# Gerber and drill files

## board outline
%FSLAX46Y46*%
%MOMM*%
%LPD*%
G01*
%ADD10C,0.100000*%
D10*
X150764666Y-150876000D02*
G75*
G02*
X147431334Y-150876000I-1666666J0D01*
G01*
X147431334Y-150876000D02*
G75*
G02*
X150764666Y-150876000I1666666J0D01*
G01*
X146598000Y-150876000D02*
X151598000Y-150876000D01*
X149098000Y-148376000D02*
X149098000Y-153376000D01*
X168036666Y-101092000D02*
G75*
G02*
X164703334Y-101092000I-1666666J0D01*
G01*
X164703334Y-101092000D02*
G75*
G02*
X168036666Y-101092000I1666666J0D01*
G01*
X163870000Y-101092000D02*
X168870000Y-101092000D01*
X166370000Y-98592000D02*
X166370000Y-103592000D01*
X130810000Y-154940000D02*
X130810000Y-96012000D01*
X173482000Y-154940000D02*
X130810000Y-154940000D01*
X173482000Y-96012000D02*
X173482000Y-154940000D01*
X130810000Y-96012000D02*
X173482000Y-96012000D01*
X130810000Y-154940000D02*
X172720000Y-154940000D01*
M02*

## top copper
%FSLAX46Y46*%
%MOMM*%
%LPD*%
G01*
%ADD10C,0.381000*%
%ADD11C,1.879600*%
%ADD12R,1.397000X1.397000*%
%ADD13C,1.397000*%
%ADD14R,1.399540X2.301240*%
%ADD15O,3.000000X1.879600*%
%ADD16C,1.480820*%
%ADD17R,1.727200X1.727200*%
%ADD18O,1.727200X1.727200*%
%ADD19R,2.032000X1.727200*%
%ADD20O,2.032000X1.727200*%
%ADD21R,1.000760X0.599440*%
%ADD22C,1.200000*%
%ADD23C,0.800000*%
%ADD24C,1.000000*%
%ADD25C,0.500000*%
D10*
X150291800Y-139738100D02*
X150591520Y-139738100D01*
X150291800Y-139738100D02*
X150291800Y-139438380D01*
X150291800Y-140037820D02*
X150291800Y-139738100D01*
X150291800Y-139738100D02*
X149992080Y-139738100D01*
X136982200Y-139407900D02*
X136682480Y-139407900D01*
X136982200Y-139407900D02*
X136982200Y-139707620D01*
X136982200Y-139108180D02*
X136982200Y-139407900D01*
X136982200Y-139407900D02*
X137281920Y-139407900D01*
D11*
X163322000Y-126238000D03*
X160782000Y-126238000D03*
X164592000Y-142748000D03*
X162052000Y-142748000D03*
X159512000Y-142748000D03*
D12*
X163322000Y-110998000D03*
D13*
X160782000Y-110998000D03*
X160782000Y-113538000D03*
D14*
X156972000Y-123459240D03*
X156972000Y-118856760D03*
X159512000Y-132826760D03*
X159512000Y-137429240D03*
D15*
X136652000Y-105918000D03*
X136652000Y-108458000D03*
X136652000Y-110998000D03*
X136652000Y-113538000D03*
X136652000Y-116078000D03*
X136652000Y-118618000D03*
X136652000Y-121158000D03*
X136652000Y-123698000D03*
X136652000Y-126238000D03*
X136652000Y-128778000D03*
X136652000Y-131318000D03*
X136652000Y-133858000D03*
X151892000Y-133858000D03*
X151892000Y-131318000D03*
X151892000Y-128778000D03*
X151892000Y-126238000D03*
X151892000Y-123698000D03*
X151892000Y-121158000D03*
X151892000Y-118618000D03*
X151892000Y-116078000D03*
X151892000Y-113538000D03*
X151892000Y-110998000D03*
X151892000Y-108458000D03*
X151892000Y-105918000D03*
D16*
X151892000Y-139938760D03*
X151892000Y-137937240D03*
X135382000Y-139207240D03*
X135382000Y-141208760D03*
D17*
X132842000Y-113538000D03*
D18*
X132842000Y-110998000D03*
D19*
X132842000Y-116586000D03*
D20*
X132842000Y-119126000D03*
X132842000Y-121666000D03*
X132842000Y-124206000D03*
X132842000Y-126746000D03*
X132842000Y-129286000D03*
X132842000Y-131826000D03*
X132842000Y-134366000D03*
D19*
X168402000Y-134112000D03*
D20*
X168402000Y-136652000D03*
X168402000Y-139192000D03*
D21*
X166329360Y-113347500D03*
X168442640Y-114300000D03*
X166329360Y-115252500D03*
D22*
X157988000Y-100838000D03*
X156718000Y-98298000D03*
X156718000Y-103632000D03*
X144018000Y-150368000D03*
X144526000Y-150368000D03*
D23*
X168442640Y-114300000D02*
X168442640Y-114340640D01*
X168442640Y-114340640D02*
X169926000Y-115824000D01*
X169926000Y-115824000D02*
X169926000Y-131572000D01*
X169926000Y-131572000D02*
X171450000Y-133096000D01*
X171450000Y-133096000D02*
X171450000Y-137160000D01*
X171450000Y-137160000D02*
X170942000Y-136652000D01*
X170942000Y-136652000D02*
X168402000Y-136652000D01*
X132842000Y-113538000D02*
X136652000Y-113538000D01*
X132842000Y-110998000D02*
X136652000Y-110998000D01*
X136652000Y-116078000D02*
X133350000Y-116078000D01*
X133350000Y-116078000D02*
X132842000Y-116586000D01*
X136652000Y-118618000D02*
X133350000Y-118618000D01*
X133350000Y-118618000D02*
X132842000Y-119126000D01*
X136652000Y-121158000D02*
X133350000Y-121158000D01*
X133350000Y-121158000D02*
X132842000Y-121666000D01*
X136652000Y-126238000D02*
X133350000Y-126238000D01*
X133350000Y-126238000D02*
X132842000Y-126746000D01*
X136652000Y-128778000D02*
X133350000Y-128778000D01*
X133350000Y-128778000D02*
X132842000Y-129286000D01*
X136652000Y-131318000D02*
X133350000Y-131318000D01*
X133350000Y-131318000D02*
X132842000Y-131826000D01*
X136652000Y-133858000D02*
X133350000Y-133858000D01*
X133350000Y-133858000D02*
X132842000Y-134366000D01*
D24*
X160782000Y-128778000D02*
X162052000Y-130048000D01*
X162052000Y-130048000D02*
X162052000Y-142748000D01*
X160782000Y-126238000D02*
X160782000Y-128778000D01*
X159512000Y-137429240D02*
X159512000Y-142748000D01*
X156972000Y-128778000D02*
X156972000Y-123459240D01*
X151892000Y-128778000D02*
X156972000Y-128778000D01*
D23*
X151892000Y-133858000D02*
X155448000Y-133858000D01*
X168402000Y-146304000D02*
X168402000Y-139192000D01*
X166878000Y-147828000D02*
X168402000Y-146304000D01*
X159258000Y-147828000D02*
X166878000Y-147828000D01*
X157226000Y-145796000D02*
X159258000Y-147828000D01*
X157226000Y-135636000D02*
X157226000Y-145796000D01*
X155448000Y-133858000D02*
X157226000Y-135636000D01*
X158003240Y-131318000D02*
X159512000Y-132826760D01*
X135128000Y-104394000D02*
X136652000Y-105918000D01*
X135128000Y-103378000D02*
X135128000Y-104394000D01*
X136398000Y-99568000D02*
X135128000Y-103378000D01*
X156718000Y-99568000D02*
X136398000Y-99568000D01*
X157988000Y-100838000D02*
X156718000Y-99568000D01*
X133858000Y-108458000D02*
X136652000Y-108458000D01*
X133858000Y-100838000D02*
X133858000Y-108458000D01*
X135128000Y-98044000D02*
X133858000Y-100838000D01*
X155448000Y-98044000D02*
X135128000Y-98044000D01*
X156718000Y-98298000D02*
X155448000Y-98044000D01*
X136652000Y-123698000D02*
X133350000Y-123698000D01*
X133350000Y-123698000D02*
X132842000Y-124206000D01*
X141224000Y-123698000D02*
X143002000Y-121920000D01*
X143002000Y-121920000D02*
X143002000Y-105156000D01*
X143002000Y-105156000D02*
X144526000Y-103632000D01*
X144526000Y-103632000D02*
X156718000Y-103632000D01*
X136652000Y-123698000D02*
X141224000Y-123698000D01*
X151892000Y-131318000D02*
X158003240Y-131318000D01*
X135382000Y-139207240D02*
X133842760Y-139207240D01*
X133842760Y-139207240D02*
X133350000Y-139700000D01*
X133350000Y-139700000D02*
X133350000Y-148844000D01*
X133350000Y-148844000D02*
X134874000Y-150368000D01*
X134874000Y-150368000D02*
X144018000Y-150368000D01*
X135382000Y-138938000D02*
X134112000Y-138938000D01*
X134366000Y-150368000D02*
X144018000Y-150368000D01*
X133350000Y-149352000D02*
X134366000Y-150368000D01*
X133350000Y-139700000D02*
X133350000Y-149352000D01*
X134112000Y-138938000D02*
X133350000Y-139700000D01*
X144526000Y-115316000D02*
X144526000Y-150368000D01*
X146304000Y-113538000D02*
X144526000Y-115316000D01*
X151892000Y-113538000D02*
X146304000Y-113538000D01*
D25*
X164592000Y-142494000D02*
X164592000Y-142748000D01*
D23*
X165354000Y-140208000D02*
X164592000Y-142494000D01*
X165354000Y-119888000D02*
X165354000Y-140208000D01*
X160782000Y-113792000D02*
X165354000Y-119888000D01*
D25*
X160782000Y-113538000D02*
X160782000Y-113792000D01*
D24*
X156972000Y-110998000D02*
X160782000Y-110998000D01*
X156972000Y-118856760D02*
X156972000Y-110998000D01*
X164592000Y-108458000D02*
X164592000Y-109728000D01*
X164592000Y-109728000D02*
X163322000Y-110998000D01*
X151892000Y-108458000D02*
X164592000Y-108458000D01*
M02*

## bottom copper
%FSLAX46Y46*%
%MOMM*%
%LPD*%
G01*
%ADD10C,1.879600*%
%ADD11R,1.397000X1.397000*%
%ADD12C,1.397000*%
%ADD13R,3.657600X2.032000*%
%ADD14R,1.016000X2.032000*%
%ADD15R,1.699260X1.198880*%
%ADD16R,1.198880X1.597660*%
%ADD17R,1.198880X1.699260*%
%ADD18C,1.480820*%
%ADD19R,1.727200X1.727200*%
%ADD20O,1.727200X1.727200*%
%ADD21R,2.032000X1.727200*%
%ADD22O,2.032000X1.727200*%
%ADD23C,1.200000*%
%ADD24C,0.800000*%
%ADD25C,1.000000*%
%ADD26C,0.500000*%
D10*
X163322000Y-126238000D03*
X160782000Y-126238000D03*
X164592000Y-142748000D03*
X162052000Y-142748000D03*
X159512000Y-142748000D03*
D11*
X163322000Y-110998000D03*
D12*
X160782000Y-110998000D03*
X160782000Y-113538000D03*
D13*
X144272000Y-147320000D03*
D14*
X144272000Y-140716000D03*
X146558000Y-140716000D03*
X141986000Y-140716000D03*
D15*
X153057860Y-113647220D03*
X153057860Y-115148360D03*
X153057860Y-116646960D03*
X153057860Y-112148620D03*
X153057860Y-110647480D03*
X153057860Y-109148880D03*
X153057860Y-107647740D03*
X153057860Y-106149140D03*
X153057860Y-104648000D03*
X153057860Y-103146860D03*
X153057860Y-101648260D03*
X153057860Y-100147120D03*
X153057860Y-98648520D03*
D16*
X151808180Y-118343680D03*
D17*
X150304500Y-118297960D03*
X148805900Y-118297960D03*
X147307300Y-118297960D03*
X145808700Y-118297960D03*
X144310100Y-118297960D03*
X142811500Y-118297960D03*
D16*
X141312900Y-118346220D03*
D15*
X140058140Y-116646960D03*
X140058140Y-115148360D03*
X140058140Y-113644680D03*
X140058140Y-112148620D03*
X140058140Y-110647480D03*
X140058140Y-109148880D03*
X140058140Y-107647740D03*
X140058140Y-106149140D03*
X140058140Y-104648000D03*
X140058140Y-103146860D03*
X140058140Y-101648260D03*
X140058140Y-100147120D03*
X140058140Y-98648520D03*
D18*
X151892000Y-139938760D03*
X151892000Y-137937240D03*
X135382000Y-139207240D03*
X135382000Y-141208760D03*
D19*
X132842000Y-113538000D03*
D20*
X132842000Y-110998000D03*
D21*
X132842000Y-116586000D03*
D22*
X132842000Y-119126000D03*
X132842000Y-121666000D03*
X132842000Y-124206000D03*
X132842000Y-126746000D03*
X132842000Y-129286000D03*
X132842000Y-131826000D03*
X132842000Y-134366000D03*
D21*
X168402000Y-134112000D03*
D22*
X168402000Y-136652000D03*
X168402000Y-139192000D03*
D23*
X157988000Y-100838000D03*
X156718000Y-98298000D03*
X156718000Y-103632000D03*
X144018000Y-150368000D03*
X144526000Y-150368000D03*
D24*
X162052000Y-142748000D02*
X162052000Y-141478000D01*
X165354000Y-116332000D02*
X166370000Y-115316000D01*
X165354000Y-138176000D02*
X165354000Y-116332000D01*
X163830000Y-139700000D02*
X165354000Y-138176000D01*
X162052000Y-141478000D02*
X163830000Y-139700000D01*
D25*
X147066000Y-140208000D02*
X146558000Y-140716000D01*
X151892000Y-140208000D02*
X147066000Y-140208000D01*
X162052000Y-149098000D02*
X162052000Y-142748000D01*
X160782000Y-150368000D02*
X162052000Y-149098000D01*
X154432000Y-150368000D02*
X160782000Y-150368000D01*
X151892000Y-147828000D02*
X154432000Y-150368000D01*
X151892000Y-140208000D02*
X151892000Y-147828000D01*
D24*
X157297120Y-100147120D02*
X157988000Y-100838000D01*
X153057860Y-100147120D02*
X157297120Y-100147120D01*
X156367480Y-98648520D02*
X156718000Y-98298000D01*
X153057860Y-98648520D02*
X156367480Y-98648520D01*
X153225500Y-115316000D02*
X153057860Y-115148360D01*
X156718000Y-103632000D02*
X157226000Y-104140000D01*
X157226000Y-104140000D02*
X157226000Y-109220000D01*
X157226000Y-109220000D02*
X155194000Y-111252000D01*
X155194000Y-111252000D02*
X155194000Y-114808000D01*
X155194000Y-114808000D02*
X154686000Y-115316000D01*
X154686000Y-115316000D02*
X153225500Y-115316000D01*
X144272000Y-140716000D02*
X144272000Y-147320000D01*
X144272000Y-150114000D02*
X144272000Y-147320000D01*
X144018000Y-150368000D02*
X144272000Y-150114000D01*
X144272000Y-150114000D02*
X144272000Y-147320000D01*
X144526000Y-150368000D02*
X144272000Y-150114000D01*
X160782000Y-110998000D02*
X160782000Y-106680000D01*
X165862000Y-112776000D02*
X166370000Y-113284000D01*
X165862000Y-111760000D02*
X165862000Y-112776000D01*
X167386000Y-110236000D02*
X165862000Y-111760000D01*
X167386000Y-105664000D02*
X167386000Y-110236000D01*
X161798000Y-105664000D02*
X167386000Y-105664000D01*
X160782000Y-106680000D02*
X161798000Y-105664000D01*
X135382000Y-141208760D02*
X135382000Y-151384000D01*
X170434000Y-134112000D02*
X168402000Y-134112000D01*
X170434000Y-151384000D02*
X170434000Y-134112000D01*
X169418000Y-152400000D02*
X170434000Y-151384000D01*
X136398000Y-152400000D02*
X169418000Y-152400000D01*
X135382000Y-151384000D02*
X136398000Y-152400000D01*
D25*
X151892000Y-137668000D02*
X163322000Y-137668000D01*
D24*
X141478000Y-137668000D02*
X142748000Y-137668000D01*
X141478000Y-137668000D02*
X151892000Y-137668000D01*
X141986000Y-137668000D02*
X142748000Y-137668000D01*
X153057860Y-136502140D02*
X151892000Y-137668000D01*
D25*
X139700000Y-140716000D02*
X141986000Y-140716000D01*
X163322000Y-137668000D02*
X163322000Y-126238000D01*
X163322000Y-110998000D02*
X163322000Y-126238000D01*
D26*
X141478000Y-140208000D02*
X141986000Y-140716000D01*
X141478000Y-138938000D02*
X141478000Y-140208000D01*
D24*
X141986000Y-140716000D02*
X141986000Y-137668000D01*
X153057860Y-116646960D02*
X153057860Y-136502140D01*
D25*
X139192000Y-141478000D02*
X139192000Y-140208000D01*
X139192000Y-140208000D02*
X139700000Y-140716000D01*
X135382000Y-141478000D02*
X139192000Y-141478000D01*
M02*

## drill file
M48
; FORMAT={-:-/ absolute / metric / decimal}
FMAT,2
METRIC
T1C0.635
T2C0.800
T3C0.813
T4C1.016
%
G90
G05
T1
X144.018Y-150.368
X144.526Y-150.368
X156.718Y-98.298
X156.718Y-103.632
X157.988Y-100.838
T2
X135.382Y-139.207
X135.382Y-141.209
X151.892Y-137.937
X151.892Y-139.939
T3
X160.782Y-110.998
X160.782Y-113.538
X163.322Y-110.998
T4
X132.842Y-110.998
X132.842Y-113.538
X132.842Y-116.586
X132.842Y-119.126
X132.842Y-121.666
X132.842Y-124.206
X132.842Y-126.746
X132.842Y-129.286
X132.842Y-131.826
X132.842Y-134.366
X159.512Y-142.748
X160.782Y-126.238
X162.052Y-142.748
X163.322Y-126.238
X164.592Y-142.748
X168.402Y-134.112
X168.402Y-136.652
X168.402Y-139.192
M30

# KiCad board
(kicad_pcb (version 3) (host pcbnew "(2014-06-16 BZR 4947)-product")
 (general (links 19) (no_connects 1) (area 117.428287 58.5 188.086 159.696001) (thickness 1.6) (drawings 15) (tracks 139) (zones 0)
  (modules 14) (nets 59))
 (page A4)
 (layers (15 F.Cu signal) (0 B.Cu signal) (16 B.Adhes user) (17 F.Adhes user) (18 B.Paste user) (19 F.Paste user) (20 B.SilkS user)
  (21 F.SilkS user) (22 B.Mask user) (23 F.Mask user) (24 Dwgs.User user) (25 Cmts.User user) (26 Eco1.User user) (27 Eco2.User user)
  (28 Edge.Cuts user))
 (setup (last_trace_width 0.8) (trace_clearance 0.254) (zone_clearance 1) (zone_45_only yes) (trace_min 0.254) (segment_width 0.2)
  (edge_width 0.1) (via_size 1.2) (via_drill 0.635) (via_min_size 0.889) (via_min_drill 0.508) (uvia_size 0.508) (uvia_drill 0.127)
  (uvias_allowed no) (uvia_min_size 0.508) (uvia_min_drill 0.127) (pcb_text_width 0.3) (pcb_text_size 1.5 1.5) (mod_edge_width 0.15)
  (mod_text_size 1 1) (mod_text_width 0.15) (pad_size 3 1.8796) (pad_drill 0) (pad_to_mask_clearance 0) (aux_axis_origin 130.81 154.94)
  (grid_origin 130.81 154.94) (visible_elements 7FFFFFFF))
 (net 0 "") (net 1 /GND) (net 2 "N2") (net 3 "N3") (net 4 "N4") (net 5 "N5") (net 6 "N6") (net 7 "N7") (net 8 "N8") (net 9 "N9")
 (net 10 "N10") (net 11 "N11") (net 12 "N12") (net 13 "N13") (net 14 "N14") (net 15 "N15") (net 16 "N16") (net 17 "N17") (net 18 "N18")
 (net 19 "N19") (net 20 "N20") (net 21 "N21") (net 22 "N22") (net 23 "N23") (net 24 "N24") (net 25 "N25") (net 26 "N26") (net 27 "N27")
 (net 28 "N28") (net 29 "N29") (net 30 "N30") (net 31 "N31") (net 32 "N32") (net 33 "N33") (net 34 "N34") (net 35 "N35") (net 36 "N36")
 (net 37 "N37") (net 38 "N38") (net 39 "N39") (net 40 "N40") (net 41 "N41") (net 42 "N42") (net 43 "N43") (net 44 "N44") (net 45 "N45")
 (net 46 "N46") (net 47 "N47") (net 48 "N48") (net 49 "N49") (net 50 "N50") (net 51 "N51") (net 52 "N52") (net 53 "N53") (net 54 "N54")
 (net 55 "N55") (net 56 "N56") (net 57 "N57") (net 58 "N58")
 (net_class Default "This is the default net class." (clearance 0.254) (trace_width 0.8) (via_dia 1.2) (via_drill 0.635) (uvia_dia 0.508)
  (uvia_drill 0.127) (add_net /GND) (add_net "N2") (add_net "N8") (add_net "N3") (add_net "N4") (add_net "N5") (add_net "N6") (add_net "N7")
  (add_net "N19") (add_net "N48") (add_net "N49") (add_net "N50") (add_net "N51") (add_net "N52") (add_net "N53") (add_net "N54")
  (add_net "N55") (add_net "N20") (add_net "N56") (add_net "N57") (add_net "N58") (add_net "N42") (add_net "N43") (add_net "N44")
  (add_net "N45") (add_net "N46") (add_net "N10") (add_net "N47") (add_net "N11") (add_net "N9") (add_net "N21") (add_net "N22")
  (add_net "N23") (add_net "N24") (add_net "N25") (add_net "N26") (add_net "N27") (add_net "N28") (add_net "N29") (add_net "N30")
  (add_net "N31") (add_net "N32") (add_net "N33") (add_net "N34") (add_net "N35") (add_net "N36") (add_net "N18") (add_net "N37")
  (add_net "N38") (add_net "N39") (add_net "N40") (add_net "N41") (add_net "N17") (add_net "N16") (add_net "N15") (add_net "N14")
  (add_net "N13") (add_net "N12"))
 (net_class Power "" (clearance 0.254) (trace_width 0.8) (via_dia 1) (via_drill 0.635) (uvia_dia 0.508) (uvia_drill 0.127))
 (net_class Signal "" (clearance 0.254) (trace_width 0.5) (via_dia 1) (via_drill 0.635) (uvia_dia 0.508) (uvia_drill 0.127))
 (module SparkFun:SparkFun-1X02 (layer F.Cu) (at 163.322 126.238 180)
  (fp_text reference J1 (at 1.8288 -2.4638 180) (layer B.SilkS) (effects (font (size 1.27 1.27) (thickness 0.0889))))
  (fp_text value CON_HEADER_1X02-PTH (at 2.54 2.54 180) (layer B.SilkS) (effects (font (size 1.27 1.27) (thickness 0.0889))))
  (pad 1 thru_hole circle (at 0 0 180) (size 1.8796 1.8796) (drill 1.016) (layers *.Cu F.Paste F.SilkS F.Mask) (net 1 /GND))
  (pad 2 thru_hole circle (at 2.54 0 180) (size 1.8796 1.8796) (drill 1.016) (layers *.Cu F.Paste F.SilkS F.Mask) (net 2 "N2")))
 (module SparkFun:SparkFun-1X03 (layer F.Cu) (at 164.592 142.748 180)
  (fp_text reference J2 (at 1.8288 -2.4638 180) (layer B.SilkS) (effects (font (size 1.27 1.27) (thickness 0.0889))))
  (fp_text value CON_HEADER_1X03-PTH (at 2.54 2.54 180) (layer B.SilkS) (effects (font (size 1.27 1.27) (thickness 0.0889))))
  (pad 1 thru_hole circle (at 0 0 180) (size 1.8796 1.8796) (drill 1.016) (layers *.Cu F.Paste F.SilkS F.Mask) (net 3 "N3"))
  (pad 2 thru_hole circle (at 2.54 0 180) (size 1.8796 1.8796) (drill 1.016) (layers *.Cu F.Paste F.SilkS F.Mask) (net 2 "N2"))
  (pad 3 thru_hole circle (at 5.08 0 180) (size 1.8796 1.8796) (drill 1.016) (layers *.Cu F.Paste F.SilkS F.Mask) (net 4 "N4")))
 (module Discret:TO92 (layer F.Cu) (at 162.052 112.268)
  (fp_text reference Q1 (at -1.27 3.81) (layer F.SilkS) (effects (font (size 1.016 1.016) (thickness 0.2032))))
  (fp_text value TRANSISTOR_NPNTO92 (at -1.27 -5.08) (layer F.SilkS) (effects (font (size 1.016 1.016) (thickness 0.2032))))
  (pad 1 thru_hole rect (at 1.27 -1.27) (size 1.397 1.397) (drill 0.8128) (layers *.Cu *.Mask F.SilkS) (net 1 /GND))
  (pad 2 thru_hole circle (at -1.27 -1.27) (size 1.397 1.397) (drill 0.8128) (layers *.Cu *.Mask F.SilkS) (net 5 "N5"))
  (pad 3 thru_hole circle (at -1.27 1.27) (size 1.397 1.397) (drill 0.8128) (layers *.Cu *.Mask F.SilkS) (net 3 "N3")))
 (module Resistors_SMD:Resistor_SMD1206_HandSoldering (layer F.Cu) (at 156.972 121.158 90)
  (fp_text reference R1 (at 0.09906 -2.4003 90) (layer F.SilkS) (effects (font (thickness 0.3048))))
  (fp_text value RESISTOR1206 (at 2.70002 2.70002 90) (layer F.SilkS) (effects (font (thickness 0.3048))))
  (pad 1 smd rect (at -2.30124 0 90) (size 2.30124 1.39954) (layers F.Cu F.Paste F.Mask) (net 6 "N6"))
  (pad 2 smd rect (at 2.30124 0 90) (size 2.30124 1.39954) (layers F.Cu F.Paste F.Mask) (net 5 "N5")))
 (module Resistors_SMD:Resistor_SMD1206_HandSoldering (layer F.Cu) (at 159.512 135.128 270)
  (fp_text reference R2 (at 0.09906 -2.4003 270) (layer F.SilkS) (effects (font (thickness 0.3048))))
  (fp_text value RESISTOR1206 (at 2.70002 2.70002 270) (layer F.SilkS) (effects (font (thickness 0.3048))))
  (pad 1 smd rect (at -2.30124 0 270) (size 2.30124 1.39954) (layers F.Cu F.Paste F.Mask) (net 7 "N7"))
  (pad 2 smd rect (at 2.30124 0 270) (size 2.30124 1.39954) (layers F.Cu F.Paste F.Mask) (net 4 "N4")))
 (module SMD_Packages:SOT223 (layer B.Cu) (at 144.272 144.018)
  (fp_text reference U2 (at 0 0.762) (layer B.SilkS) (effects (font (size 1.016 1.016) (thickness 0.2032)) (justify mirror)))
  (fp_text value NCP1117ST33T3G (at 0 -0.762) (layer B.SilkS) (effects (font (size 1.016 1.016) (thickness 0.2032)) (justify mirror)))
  (pad 4 smd rect (at 0 3.302) (size 3.6576 2.032) (layers B.Cu B.Paste B.Mask))
  (pad 2 smd rect (at 0 -3.302) (size 1.016 2.032) (layers B.Cu B.Paste B.Mask) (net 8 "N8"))
  (pad 3 smd rect (at 2.286 -3.302) (size 1.016 2.032) (layers B.Cu B.Paste B.Mask) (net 2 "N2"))
  (pad 1 smd rect (at -2.286 -3.302) (size 1.016 2.032) (layers B.Cu B.Paste B.Mask) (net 1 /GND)))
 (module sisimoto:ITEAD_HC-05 (layer B.Cu) (at 146.558 104.648 180)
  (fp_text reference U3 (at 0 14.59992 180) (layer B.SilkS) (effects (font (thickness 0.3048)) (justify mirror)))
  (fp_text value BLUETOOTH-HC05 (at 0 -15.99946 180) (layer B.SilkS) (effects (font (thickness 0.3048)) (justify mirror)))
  (pad 11 smd rect (at -6.49986 -8.99922 180) (size 1.69926 1.19888) (layers B.Cu B.Paste B.Mask) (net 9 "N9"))
  (pad 12 smd rect (at -6.49986 -10.50036 180) (size 1.69926 1.19888) (layers B.Cu B.Paste B.Mask) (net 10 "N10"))
  (pad 13 smd rect (at -6.49986 -11.99896 180) (size 1.69926 1.19888) (layers B.Cu B.Paste B.Mask) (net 1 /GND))
  (pad 10 smd rect (at -6.49986 -7.50062 180) (size 1.69926 1.19888) (layers B.Cu B.Paste B.Mask) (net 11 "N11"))
  (pad 9 smd rect (at -6.49986 -5.99948 180) (size 1.69926 1.19888) (layers B.Cu B.Paste B.Mask) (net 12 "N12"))
  (pad 8 smd rect (at -6.49986 -4.50088 180) (size 1.69926 1.19888) (layers B.Cu B.Paste B.Mask) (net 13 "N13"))
  (pad 7 smd rect (at -6.49986 -2.99974 180) (size 1.69926 1.19888) (layers B.Cu B.Paste B.Mask) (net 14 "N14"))
  (pad 6 smd rect (at -6.49986 -1.50114 180) (size 1.69926 1.19888) (layers B.Cu B.Paste B.Mask) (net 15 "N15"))
  (pad 5 smd rect (at -6.49986 0 180) (size 1.69926 1.19888) (layers B.Cu B.Paste B.Mask) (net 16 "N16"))
  (pad 4 smd rect (at -6.49986 1.50114 180) (size 1.69926 1.19888) (layers B.Cu B.Paste B.Mask) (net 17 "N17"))
  (pad 3 smd rect (at -6.49986 2.99974 180) (size 1.69926 1.19888) (layers B.Cu B.Paste B.Mask) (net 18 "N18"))
  (pad 2 smd rect (at -6.49986 4.50088 180) (size 1.69926 1.19888) (layers B.Cu B.Paste B.Mask) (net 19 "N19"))
  (pad 1 smd rect (at -6.49986 5.99948 180) (size 1.69926 1.19888) (layers B.Cu B.Paste B.Mask) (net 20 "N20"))
  (pad 14 smd rect (at -5.25018 -13.69568 180) (size 1.19888 1.59766) (layers B.Cu B.Paste B.Mask) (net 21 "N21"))
  (pad 15 smd rect (at -3.7465 -13.64996 180) (size 1.19888 1.69926) (layers B.Cu B.Paste B.Mask) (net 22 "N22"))
  (pad 16 smd rect (at -2.2479 -13.64996 180) (size 1.19888 1.69926) (layers B.Cu B.Paste B.Mask) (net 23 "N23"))
  (pad 17 smd rect (at -0.7493 -13.64996 180) (size 1.19888 1.69926) (layers B.Cu B.Paste B.Mask) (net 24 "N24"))
  (pad 18 smd rect (at 0.7493 -13.64996 180) (size 1.19888 1.69926) (layers B.Cu B.Paste B.Mask) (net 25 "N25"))
  (pad 19 smd rect (at 2.2479 -13.64996 180) (size 1.19888 1.69926) (layers B.Cu B.Paste B.Mask) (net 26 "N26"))
  (pad 20 smd rect (at 3.7465 -13.64996 180) (size 1.19888 1.69926) (layers B.Cu B.Paste B.Mask) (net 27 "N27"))
  (pad 21 smd rect (at 5.2451 -13.69822 180) (size 1.19888 1.59766) (layers B.Cu B.Paste B.Mask) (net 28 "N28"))
  (pad 22 smd rect (at 6.49986 -11.99896 180) (size 1.69926 1.19888) (layers B.Cu B.Paste B.Mask) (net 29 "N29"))
  (pad 23 smd rect (at 6.49986 -10.50036 180) (size 1.69926 1.19888) (layers B.Cu B.Paste B.Mask) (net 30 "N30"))
  (pad 24 smd rect (at 6.49986 -8.99668 180) (size 1.69926 1.19888) (layers B.Cu B.Paste B.Mask) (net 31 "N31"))
  (pad 25 smd rect (at 6.49986 -7.50062 180) (size 1.69926 1.19888) (layers B.Cu B.Paste B.Mask) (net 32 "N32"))
  (pad 26 smd rect (at 6.49986 -5.99948 180) (size 1.69926 1.19888) (layers B.Cu B.Paste B.Mask) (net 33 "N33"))
  (pad 27 smd rect (at 6.49986 -4.50088 180) (size 1.69926 1.19888) (layers B.Cu B.Paste B.Mask) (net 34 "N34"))
  (pad 28 smd rect (at 6.49986 -2.99974 180) (size 1.69926 1.19888) (layers B.Cu B.Paste B.Mask) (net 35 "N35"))
  (pad 29 smd rect (at 6.49986 -1.50114 180) (size 1.69926 1.19888) (layers B.Cu B.Paste B.Mask) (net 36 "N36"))
  (pad 30 smd rect (at 6.49986 0 180) (size 1.69926 1.19888) (layers B.Cu B.Paste B.Mask) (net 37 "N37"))
  (pad 31 smd rect (at 6.49986 1.50114 180) (size 1.69926 1.19888) (layers B.Cu B.Paste B.Mask) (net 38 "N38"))
  (pad 32 smd rect (at 6.49986 2.99974 180) (size 1.69926 1.19888) (layers B.Cu B.Paste B.Mask) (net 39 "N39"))
  (pad 33 smd rect (at 6.49986 4.50088 180) (size 1.69926 1.19888) (layers B.Cu B.Paste B.Mask) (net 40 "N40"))
  (pad 34 smd rect (at 6.49986 5.99948 180) (size 1.69926 1.19888) (layers B.Cu B.Paste B.Mask) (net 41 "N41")))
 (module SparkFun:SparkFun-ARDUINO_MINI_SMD (layer F.Cu) (at 144.272 118.618)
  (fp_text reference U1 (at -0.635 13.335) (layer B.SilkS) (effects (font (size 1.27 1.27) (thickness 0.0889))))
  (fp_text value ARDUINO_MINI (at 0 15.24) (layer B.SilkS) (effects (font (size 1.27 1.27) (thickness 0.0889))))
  (pad 1 smd oval (at -7.62 -12.7) (size 3 1.8796) (layers F.Cu F.Paste F.Mask) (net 19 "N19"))
  (pad 2 smd oval (at -7.62 -10.16) (size 3 1.8796) (layers F.Cu F.Paste F.Mask) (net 20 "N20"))
  (pad 3 smd oval (at -7.62 -7.62) (size 3 1.8796) (layers F.Cu F.Paste F.Mask) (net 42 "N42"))
  (pad 4 smd oval (at -7.62 -5.08) (size 3 1.8796) (layers F.Cu F.Paste F.Mask) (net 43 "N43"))
  (pad 5 smd oval (at -7.62 -2.54) (size 3 1.8796) (layers F.Cu F.Paste F.Mask) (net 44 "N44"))
  (pad 6 smd oval (at -7.62 0) (size 3 1.8796) (layers F.Cu F.Paste F.Mask) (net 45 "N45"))
  (pad 7 smd oval (at -7.62 2.54) (size 3 1.8796) (layers F.Cu F.Paste F.Mask) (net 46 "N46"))
  (pad 8 smd oval (at -7.62 5.08) (size 3 1.8796) (layers F.Cu F.Paste F.Mask) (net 10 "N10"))
  (pad 9 smd oval (at -7.62 7.62) (size 3 1.8796) (layers F.Cu F.Paste F.Mask) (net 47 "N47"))
  (pad 10 smd oval (at -7.62 10.16) (size 3 1.8796) (layers F.Cu F.Paste F.Mask) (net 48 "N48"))
  (pad 11 smd oval (at -7.62 12.7) (size 3 1.8796) (layers F.Cu F.Paste F.Mask) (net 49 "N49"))
  (pad 12 smd oval (at -7.62 15.24) (size 3 1.8796) (layers F.Cu F.Paste F.Mask) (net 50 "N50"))
  (pad 13 smd oval (at 7.62 15.24) (size 3 1.8796) (layers F.Cu F.Paste F.Mask) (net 7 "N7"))
  (pad 14 smd oval (at 7.62 12.7) (size 3 1.8796) (layers F.Cu F.Paste F.Mask) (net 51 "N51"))
  (pad 15 smd oval (at 7.62 10.16) (size 3 1.8796) (layers F.Cu F.Paste F.Mask) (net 6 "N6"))
  (pad 16 smd oval (at 7.62 7.62) (size 3 1.8796) (layers F.Cu F.Paste F.Mask) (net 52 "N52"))
  (pad 17 smd oval (at 7.62 5.08) (size 3 1.8796) (layers F.Cu F.Paste F.Mask) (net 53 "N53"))
  (pad 18 smd oval (at 7.62 2.54) (size 3 1.8796) (layers F.Cu F.Paste F.Mask) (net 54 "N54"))
  (pad 19 smd oval (at 7.62 0) (size 3 1.8796) (layers F.Cu F.Paste F.Mask) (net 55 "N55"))
  (pad 20 smd oval (at 7.62 -2.54) (size 3 1.8796) (layers F.Cu F.Paste F.Mask) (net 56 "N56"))
  (pad 21 smd oval (at 7.62 -5.08) (size 3 1.8796) (layers F.Cu F.Paste F.Mask) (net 8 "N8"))
  (pad 22 smd oval (at 7.62 -7.62) (size 3 1.8796) (layers F.Cu F.Paste F.Mask) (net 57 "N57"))
  (pad 23 smd oval (at 7.62 -10.16) (size 3 1.8796) (layers F.Cu F.Paste F.Mask) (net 1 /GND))
  (pad 24 smd oval (at 7.62 -12.7) (size 3 1.8796) (layers F.Cu F.Paste F.Mask) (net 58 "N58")))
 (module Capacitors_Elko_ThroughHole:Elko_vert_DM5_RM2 (layer F.Cu) (at 151.892 138.938 90)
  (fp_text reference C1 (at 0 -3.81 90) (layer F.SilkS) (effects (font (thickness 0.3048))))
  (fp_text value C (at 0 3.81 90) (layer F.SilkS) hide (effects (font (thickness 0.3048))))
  (fp_line (start -0.8001 -1.6002) (end -0.8001 -1.30048) (layer F.Cu) (width 0.381))
  (fp_line (start -0.8001 -1.6002) (end -0.50038 -1.6002) (layer F.Cu) (width 0.381))
  (fp_line (start -1.09982 -1.6002) (end -0.8001 -1.6002) (layer F.Cu) (width 0.381))
  (fp_line (start -0.8001 -1.6002) (end -0.8001 -1.89992) (layer F.Cu) (width 0.381))
  (pad 1 thru_hole circle (at -1.00076 0 90) (size 1.48082 1.48082) (drill 0.8001) (layers *.Cu *.Mask F.SilkS) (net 2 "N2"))
  (pad 2 thru_hole circle (at 1.00076 0 90) (size 1.48082 1.48082) (drill 0.8001) (layers *.Cu *.Mask F.SilkS) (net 1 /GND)))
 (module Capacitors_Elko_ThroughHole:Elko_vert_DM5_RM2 (layer F.Cu) (at 135.382 140.208 270)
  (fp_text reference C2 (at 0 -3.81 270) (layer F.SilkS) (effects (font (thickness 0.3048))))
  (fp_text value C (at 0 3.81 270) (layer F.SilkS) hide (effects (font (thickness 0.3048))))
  (fp_line (start -0.8001 -1.6002) (end -0.8001 -1.30048) (layer F.Cu) (width 0.381))
  (fp_line (start -0.8001 -1.6002) (end -0.50038 -1.6002) (layer F.Cu) (width 0.381))
  (fp_line (start -1.09982 -1.6002) (end -0.8001 -1.6002) (layer F.Cu) (width 0.381))
  (fp_line (start -0.8001 -1.6002) (end -0.8001 -1.89992) (layer F.Cu) (width 0.381))
  (pad 1 thru_hole circle (at -1.00076 0 270) (size 1.48082 1.48082) (drill 0.8001) (layers *.Cu *.Mask F.SilkS) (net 8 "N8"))
  (pad 2 thru_hole circle (at 1.00076 0 270) (size 1.48082 1.48082) (drill 0.8001) (layers *.Cu *.Mask F.SilkS) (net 1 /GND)))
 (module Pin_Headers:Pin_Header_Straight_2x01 (layer F.Cu) (at 132.842 112.268)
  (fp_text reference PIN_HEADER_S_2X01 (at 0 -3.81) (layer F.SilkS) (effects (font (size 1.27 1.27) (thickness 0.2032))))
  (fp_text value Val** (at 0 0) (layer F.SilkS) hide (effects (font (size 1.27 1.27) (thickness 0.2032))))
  (pad 1 thru_hole rect (at 0 1.27) (size 1.7272 1.7272) (drill 1.016) (layers *.Cu *.Mask F.SilkS))
  (pad 2 thru_hole oval (at 0 -1.27) (size 1.7272 1.7272) (drill 1.016) (layers *.Cu *.Mask F.SilkS)))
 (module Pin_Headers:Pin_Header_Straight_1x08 (layer F.Cu) (at 132.842 125.476 270)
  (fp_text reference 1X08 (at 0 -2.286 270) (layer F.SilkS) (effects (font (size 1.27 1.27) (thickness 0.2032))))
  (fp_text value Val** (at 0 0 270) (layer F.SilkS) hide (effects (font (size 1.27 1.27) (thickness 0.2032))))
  (pad 1 thru_hole rect (at -8.89 0 270) (size 1.7272 2.032) (drill 1.016) (layers *.Cu *.Mask F.SilkS))
  (pad 2 thru_hole oval (at -6.35 0 270) (size 1.7272 2.032) (drill 1.016) (layers *.Cu *.Mask F.SilkS))
  (pad 3 thru_hole oval (at -3.81 0 270) (size 1.7272 2.032) (drill 1.016) (layers *.Cu *.Mask F.SilkS))
  (pad 4 thru_hole oval (at -1.27 0 270) (size 1.7272 2.032) (drill 1.016) (layers *.Cu *.Mask F.SilkS))
  (pad 5 thru_hole oval (at 1.27 0 270) (size 1.7272 2.032) (drill 1.016) (layers *.Cu *.Mask F.SilkS))
  (pad 6 thru_hole oval (at 3.81 0 270) (size 1.7272 2.032) (drill 1.016) (layers *.Cu *.Mask F.SilkS))
  (pad 7 thru_hole oval (at 6.35 0 270) (size 1.7272 2.032) (drill 1.016) (layers *.Cu *.Mask F.SilkS))
  (pad 8 thru_hole oval (at 8.89 0 270) (size 1.7272 2.032) (drill 1.016) (layers *.Cu *.Mask F.SilkS)))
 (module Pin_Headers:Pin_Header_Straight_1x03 (layer F.Cu) (at 168.402 136.652 270)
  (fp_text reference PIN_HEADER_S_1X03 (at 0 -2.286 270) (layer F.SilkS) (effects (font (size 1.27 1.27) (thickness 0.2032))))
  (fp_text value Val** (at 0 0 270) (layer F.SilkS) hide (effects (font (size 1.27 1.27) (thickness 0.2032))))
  (pad 1 thru_hole rect (at -2.54 0 270) (size 1.7272 2.032) (drill 1.016) (layers *.Cu *.Mask F.SilkS))
  (pad 2 thru_hole oval (at 0 0 270) (size 1.7272 2.032) (drill 1.016) (layers *.Cu *.Mask F.SilkS))
  (pad 3 thru_hole oval (at 2.54 0 270) (size 1.7272 2.032) (drill 1.016) (layers *.Cu *.Mask F.SilkS)))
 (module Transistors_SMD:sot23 (layer F.Cu) (at 167.386 114.3 270)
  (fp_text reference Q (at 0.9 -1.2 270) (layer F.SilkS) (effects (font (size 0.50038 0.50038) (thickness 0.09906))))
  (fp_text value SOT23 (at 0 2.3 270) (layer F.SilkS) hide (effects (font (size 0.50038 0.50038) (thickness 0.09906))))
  (pad 1 smd rect (at -0.9525 1.05664 270) (size 0.59944 1.00076) (layers F.Cu F.Paste F.Mask))
  (pad 3 smd rect (at 0 -1.05664 270) (size 0.59944 1.00076) (layers F.Cu F.Paste F.Mask))
  (pad 2 smd rect (at 0.9525 1.05664 270) (size 0.59944 1.00076) (layers F.Cu F.Paste F.Mask)))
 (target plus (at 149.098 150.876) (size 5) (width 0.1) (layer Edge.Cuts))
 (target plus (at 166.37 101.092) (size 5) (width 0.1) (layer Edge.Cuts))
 (gr_line (start 130.81 154.94) (end 130.81 96.012) (angle 90) (layer Edge.Cuts) (width 0.1))
 (gr_line (start 173.482 154.94) (end 130.81 154.94) (angle 90) (layer Edge.Cuts) (width 0.1))
 (gr_line (start 173.482 96.012) (end 173.482 154.94) (angle 90) (layer Edge.Cuts) (width 0.1))
 (gr_line (start 130.81 96.012) (end 173.482 96.012) (angle 90) (layer Edge.Cuts) (width 0.1))
 (gr_line (start 130.81 154.94) (end 172.72 154.94) (angle 90) (layer Edge.Cuts) (width 0.1))
 (segment (start 168.44264 114.3) (end 168.44264 114.34064) (width 0.8) (layer F.Cu) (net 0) (status C00000))
 (segment (start 168.44264 114.34064) (end 169.926 115.824) (width 0.8) (layer F.Cu) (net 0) (status 400000))
 (segment (start 169.926 115.824) (end 169.926 131.572) (width 0.8) (layer F.Cu) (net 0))
 (segment (start 169.926 131.572) (end 171.45 133.096) (width 0.8) (layer F.Cu) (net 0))
 (segment (start 171.45 133.096) (end 171.45 137.16) (width 0.8) (layer F.Cu) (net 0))
 (segment (start 171.45 137.16) (end 170.942 136.652) (width 0.8) (layer F.Cu) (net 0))
 (segment (start 170.942 136.652) (end 168.402 136.652) (width 0.8) (layer F.Cu) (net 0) (status 800000))
 (segment (start 132.842 113.538) (end 136.652 113.538) (width 0.8) (layer F.Cu) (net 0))
 (segment (start 132.842 110.998) (end 136.652 110.998) (width 0.8) (layer F.Cu) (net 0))
 (segment (start 136.652 116.078) (end 133.35 116.078) (width 0.8) (layer F.Cu) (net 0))
 (segment (start 133.35 116.078) (end 132.842 116.586) (width 0.8) (layer F.Cu) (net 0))
 (segment (start 136.652 118.618) (end 133.35 118.618) (width 0.8) (layer F.Cu) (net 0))
 (segment (start 133.35 118.618) (end 132.842 119.126) (width 0.8) (layer F.Cu) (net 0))
 (segment (start 136.652 121.158) (end 133.35 121.158) (width 0.8) (layer F.Cu) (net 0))
 (segment (start 133.35 121.158) (end 132.842 121.666) (width 0.8) (layer F.Cu) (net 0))
 (segment (start 136.652 126.238) (end 133.35 126.238) (width 0.8) (layer F.Cu) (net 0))
 (segment (start 133.35 126.238) (end 132.842 126.746) (width 0.8) (layer F.Cu) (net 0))
 (segment (start 136.652 128.778) (end 133.35 128.778) (width 0.8) (layer F.Cu) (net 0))
 (segment (start 133.35 128.778) (end 132.842 129.286) (width 0.8) (layer F.Cu) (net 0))
 (segment (start 136.652 131.318) (end 133.35 131.318) (width 0.8) (layer F.Cu) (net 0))
 (segment (start 133.35 131.318) (end 132.842 131.826) (width 0.8) (layer F.Cu) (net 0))
 (segment (start 136.652 133.858) (end 133.35 133.858) (width 0.8) (layer F.Cu) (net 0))
 (segment (start 133.35 133.858) (end 132.842 134.366) (width 0.8) (layer F.Cu) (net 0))
 (segment (start 162.052 142.748) (end 162.052 141.478) (width 0.8) (layer B.Cu) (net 2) (status 400000))
 (segment (start 165.354 116.332) (end 166.37 115.316) (width 0.8) (layer B.Cu) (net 2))
 (segment (start 165.354 138.176) (end 165.354 116.332) (width 0.8) (layer B.Cu) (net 2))
 (segment (start 163.83 139.7) (end 165.354 138.176) (width 0.8) (layer B.Cu) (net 2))
 (segment (start 162.052 141.478) (end 163.83 139.7) (width 0.8) (layer B.Cu) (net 2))
 (segment (start 147.066 140.208) (end 146.558 140.716) (width 1) (layer B.Cu) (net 2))
 (segment (start 151.892 140.208) (end 147.066 140.208) (width 1) (layer B.Cu) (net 2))
 (segment (start 162.052 149.098) (end 162.052 142.748) (width 1) (layer B.Cu) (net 2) (status 20))
 (segment (start 160.782 128.778) (end 162.052 130.048) (width 1) (layer F.Cu) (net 2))
 (segment (start 162.052 130.048) (end 162.052 142.748) (width 1) (layer F.Cu) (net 2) (status 20))
 (segment (start 160.782 126.238) (end 160.782 128.778) (width 1) (layer F.Cu) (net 2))
 (segment (start 160.782 150.368) (end 162.052 149.098) (width 1) (layer B.Cu) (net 2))
 (segment (start 154.432 150.368) (end 160.782 150.368) (width 1) (layer B.Cu) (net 2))
 (segment (start 151.892 147.828) (end 154.432 150.368) (width 1) (layer B.Cu) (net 2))
 (segment (start 151.892 140.208) (end 151.892 147.828) (width 1) (layer B.Cu) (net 2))
 (segment (start 159.512 137.42924) (end 159.512 142.748) (width 1) (layer F.Cu) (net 4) (status 20))
 (segment (start 156.972 128.778) (end 156.972 123.45924) (width 1) (layer F.Cu) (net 6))
 (segment (start 151.892 128.778) (end 156.972 128.778) (width 1) (layer F.Cu) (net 6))
 (segment (start 151.892 133.858) (end 155.448 133.858) (width 0.8) (layer F.Cu) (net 7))
 (segment (start 168.402 146.304) (end 168.402 139.192) (width 0.8) (layer F.Cu) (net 7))
 (segment (start 166.878 147.828) (end 168.402 146.304) (width 0.8) (layer F.Cu) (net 7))
 (segment (start 159.258 147.828) (end 166.878 147.828) (width 0.8) (layer F.Cu) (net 7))
 (segment (start 157.226 145.796) (end 159.258 147.828) (width 0.8) (layer F.Cu) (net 7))
 (segment (start 157.226 135.636) (end 157.226 145.796) (width 0.8) (layer F.Cu) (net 7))
 (segment (start 155.448 133.858) (end 157.226 135.636) (width 0.8) (layer F.Cu) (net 7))
 (segment (start 158.00324 131.318) (end 159.512 132.82676) (width 0.8) (layer F.Cu) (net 7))
 (segment (start 135.128 104.394) (end 136.652 105.918) (width 0.8) (layer F.Cu) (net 19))
 (segment (start 135.128 103.378) (end 135.128 104.394) (width 0.8) (layer F.Cu) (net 19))
 (segment (start 136.398 99.568) (end 135.128 103.378) (width 0.8) (layer F.Cu) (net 19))
 (segment (start 156.718 99.568) (end 136.398 99.568) (width 0.8) (layer F.Cu) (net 19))
 (segment (start 157.988 100.838) (end 156.718 99.568) (width 0.8) (layer F.Cu) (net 19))
 (via (at 157.988 100.838) (size 1.2) (layers F.Cu B.Cu) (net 19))
 (segment (start 157.29712 100.14712) (end 157.988 100.838) (width 0.8) (layer B.Cu) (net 19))
 (segment (start 153.05786 100.14712) (end 157.29712 100.14712) (width 0.8) (layer B.Cu) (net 19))
 (segment (start 133.858 108.458) (end 136.652 108.458) (width 0.8) (layer F.Cu) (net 20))
 (segment (start 133.858 100.838) (end 133.858 108.458) (width 0.8) (layer F.Cu) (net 20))
 (segment (start 135.128 98.044) (end 133.858 100.838) (width 0.8) (layer F.Cu) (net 20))
 (segment (start 155.448 98.044) (end 135.128 98.044) (width 0.8) (layer F.Cu) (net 20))
 (segment (start 156.718 98.298) (end 155.448 98.044) (width 0.8) (layer F.Cu) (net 20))
 (via (at 156.718 98.298) (size 1.2) (layers F.Cu B.Cu) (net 20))
 (segment (start 156.36748 98.64852) (end 156.718 98.298) (width 0.8) (layer B.Cu) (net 20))
 (segment (start 153.05786 98.64852) (end 156.36748 98.64852) (width 0.8) (layer B.Cu) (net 20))
 (segment (start 136.652 123.698) (end 133.35 123.698) (width 0.8) (layer F.Cu) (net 10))
 (segment (start 133.35 123.698) (end 132.842 124.206) (width 0.8) (layer F.Cu) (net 10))
 (segment (start 153.2255 115.316) (end 153.05786 115.14836) (width 0.8) (layer B.Cu) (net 10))
 (segment (start 141.224 123.698) (end 143.002 121.92) (width 0.8) (layer F.Cu) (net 10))
 (segment (start 143.002 121.92) (end 143.002 105.156) (width 0.8) (layer F.Cu) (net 10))
 (segment (start 143.002 105.156) (end 144.526 103.632) (width 0.8) (layer F.Cu) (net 10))
 (segment (start 144.526 103.632) (end 156.718 103.632) (width 0.8) (layer F.Cu) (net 10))
 (via (at 156.718 103.632) (size 1.2) (layers F.Cu B.Cu) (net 10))
 (segment (start 156.718 103.632) (end 157.226 104.14) (width 0.8) (layer B.Cu) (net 10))
 (segment (start 157.226 104.14) (end 157.226 109.22) (width 0.8) (layer B.Cu) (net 10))
 (segment (start 157.226 109.22) (end 155.194 111.252) (width 0.8) (layer B.Cu) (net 10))
 (segment (start 155.194 111.252) (end 155.194 114.808) (width 0.8) (layer B.Cu) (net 10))
 (segment (start 155.194 114.808) (end 154.686 115.316) (width 0.8) (layer B.Cu) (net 10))
 (segment (start 154.686 115.316) (end 153.2255 115.316) (width 0.8) (layer B.Cu) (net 10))
 (segment (start 136.652 123.698) (end 141.224 123.698) (width 0.8) (layer F.Cu) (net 10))
 (segment (start 151.892 131.318) (end 158.00324 131.318) (width 0.8) (layer F.Cu) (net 51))
 (segment (start 135.382 139.20724) (end 133.84276 139.20724) (width 0.8) (layer F.Cu) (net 8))
 (segment (start 133.84276 139.20724) (end 133.35 139.7) (width 0.8) (layer F.Cu) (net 8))
 (segment (start 133.35 139.7) (end 133.35 148.844) (width 0.8) (layer F.Cu) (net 8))
 (segment (start 133.35 148.844) (end 134.874 150.368) (width 0.8) (layer F.Cu) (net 8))
 (segment (start 134.874 150.368) (end 144.018 150.368) (width 0.8) (layer F.Cu) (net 8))
 (segment (start 135.382 138.938) (end 134.112 138.938) (width 0.8) (layer F.Cu) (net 8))
 (segment (start 144.272 140.716) (end 144.272 147.32) (width 0.8) (layer B.Cu) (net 8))
 (segment (start 144.272 150.114) (end 144.272 147.32) (width 0.8) (layer B.Cu) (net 8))
 (segment (start 144.018 150.368) (end 144.272 150.114) (width 0.8) (layer B.Cu) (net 8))
 (via (at 144.018 150.368) (size 1.2) (layers F.Cu B.Cu) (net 8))
 (segment (start 134.366 150.368) (end 144.018 150.368) (width 0.8) (layer F.Cu) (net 8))
 (segment (start 133.35 149.352) (end 134.366 150.368) (width 0.8) (layer F.Cu) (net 8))
 (segment (start 133.35 139.7) (end 133.35 149.352) (width 0.8) (layer F.Cu) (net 8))
 (segment (start 134.112 138.938) (end 133.35 139.7) (width 0.8) (layer F.Cu) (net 8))
 (segment (start 144.272 150.114) (end 144.272 147.32) (width 0.8) (layer B.Cu) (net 8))
 (segment (start 144.526 150.368) (end 144.272 150.114) (width 0.8) (layer B.Cu) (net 8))
 (via (at 144.526 150.368) (size 1.2) (layers F.Cu B.Cu) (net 8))
 (segment (start 144.526 115.316) (end 144.526 150.368) (width 0.8) (layer F.Cu) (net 8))
 (segment (start 146.304 113.538) (end 144.526 115.316) (width 0.8) (layer F.Cu) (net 8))
 (segment (start 151.892 113.538) (end 146.304 113.538) (width 0.8) (layer F.Cu) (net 8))
 (segment (start 164.592 142.494) (end 164.592 142.748) (width 0.5) (layer F.Cu) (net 3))
 (segment (start 165.354 140.208) (end 164.592 142.494) (width 0.8) (layer F.Cu) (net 3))
 (segment (start 165.354 119.888) (end 165.354 140.208) (width 0.8) (layer F.Cu) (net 3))
 (segment (start 160.782 113.792) (end 165.354 119.888) (width 0.8) (layer F.Cu) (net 3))
 (segment (start 160.782 113.538) (end 160.782 113.792) (width 0.5) (layer F.Cu) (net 3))
 (segment (start 160.782 110.998) (end 160.782 106.68) (width 0.8) (layer B.Cu) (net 5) (status 400000))
 (segment (start 165.862 112.776) (end 166.37 113.284) (width 0.8) (layer B.Cu) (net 5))
 (segment (start 165.862 111.76) (end 165.862 112.776) (width 0.8) (layer B.Cu) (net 5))
 (segment (start 167.386 110.236) (end 165.862 111.76) (width 0.8) (layer B.Cu) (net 5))
 (segment (start 167.386 105.664) (end 167.386 110.236) (width 0.8) (layer B.Cu) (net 5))
 (segment (start 161.798 105.664) (end 167.386 105.664) (width 0.8) (layer B.Cu) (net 5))
 (segment (start 160.782 106.68) (end 161.798 105.664) (width 0.8) (layer B.Cu) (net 5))
 (segment (start 156.972 110.998) (end 160.782 110.998) (width 1) (layer F.Cu) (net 5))
 (segment (start 156.972 118.85676) (end 156.972 110.998) (width 1) (layer F.Cu) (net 5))
 (segment (start 135.382 141.20876) (end 135.382 151.384) (width 0.8) (layer B.Cu) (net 1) (status 400000))
 (segment (start 170.434 134.112) (end 168.402 134.112) (width 0.8) (layer B.Cu) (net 1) (status 800000))
 (segment (start 170.434 151.384) (end 170.434 134.112) (width 0.8) (layer B.Cu) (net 1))
 (segment (start 169.418 152.4) (end 170.434 151.384) (width 0.8) (layer B.Cu) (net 1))
 (segment (start 136.398 152.4) (end 169.418 152.4) (width 0.8) (layer B.Cu) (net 1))
 (segment (start 135.382 151.384) (end 136.398 152.4) (width 0.8) (layer B.Cu) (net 1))
 (segment (start 151.892 137.668) (end 163.322 137.668) (width 1) (layer B.Cu) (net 1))
 (segment (start 141.478 137.668) (end 142.748 137.668) (width 0.8) (layer B.Cu) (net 1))
 (segment (start 141.478 137.668) (end 151.892 137.668) (width 0.8) (layer B.Cu) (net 1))
 (segment (start 141.986 137.668) (end 142.748 137.668) (width 0.8) (layer B.Cu) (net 1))
 (segment (start 153.05786 136.50214) (end 151.892 137.668) (width 0.8) (layer B.Cu) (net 1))
 (segment (start 139.7 140.716) (end 141.986 140.716) (width 1) (layer B.Cu) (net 1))
 (segment (start 163.322 137.668) (end 163.322 126.238) (width 1) (layer B.Cu) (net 1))
 (segment (start 164.592 108.458) (end 164.592 109.728) (width 1) (layer F.Cu) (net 1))
 (segment (start 164.592 109.728) (end 163.322 110.998) (width 1) (layer F.Cu) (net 1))
 (segment (start 151.892 108.458) (end 164.592 108.458) (width 1) (layer F.Cu) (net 1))
 (segment (start 163.322 110.998) (end 163.322 126.238) (width 1) (layer B.Cu) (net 1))
 (segment (start 141.478 140.208) (end 141.986 140.716) (width 0.5) (layer B.Cu) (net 1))
 (segment (start 141.478 138.938) (end 141.478 140.208) (width 0.5) (layer B.Cu) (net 1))
 (segment (start 141.986 140.716) (end 141.986 137.668) (width 0.8) (layer B.Cu) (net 1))
 (segment (start 153.05786 116.64696) (end 153.05786 136.50214) (width 0.8) (layer B.Cu) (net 1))
 (segment (start 139.192 141.478) (end 139.192 140.208) (width 1) (layer B.Cu) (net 1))
 (segment (start 139.192 140.208) (end 139.7 140.716) (width 1) (layer B.Cu) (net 1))
 (segment (start 135.382 141.478) (end 139.192 141.478) (width 1) (layer B.Cu) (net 1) (status 10)))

